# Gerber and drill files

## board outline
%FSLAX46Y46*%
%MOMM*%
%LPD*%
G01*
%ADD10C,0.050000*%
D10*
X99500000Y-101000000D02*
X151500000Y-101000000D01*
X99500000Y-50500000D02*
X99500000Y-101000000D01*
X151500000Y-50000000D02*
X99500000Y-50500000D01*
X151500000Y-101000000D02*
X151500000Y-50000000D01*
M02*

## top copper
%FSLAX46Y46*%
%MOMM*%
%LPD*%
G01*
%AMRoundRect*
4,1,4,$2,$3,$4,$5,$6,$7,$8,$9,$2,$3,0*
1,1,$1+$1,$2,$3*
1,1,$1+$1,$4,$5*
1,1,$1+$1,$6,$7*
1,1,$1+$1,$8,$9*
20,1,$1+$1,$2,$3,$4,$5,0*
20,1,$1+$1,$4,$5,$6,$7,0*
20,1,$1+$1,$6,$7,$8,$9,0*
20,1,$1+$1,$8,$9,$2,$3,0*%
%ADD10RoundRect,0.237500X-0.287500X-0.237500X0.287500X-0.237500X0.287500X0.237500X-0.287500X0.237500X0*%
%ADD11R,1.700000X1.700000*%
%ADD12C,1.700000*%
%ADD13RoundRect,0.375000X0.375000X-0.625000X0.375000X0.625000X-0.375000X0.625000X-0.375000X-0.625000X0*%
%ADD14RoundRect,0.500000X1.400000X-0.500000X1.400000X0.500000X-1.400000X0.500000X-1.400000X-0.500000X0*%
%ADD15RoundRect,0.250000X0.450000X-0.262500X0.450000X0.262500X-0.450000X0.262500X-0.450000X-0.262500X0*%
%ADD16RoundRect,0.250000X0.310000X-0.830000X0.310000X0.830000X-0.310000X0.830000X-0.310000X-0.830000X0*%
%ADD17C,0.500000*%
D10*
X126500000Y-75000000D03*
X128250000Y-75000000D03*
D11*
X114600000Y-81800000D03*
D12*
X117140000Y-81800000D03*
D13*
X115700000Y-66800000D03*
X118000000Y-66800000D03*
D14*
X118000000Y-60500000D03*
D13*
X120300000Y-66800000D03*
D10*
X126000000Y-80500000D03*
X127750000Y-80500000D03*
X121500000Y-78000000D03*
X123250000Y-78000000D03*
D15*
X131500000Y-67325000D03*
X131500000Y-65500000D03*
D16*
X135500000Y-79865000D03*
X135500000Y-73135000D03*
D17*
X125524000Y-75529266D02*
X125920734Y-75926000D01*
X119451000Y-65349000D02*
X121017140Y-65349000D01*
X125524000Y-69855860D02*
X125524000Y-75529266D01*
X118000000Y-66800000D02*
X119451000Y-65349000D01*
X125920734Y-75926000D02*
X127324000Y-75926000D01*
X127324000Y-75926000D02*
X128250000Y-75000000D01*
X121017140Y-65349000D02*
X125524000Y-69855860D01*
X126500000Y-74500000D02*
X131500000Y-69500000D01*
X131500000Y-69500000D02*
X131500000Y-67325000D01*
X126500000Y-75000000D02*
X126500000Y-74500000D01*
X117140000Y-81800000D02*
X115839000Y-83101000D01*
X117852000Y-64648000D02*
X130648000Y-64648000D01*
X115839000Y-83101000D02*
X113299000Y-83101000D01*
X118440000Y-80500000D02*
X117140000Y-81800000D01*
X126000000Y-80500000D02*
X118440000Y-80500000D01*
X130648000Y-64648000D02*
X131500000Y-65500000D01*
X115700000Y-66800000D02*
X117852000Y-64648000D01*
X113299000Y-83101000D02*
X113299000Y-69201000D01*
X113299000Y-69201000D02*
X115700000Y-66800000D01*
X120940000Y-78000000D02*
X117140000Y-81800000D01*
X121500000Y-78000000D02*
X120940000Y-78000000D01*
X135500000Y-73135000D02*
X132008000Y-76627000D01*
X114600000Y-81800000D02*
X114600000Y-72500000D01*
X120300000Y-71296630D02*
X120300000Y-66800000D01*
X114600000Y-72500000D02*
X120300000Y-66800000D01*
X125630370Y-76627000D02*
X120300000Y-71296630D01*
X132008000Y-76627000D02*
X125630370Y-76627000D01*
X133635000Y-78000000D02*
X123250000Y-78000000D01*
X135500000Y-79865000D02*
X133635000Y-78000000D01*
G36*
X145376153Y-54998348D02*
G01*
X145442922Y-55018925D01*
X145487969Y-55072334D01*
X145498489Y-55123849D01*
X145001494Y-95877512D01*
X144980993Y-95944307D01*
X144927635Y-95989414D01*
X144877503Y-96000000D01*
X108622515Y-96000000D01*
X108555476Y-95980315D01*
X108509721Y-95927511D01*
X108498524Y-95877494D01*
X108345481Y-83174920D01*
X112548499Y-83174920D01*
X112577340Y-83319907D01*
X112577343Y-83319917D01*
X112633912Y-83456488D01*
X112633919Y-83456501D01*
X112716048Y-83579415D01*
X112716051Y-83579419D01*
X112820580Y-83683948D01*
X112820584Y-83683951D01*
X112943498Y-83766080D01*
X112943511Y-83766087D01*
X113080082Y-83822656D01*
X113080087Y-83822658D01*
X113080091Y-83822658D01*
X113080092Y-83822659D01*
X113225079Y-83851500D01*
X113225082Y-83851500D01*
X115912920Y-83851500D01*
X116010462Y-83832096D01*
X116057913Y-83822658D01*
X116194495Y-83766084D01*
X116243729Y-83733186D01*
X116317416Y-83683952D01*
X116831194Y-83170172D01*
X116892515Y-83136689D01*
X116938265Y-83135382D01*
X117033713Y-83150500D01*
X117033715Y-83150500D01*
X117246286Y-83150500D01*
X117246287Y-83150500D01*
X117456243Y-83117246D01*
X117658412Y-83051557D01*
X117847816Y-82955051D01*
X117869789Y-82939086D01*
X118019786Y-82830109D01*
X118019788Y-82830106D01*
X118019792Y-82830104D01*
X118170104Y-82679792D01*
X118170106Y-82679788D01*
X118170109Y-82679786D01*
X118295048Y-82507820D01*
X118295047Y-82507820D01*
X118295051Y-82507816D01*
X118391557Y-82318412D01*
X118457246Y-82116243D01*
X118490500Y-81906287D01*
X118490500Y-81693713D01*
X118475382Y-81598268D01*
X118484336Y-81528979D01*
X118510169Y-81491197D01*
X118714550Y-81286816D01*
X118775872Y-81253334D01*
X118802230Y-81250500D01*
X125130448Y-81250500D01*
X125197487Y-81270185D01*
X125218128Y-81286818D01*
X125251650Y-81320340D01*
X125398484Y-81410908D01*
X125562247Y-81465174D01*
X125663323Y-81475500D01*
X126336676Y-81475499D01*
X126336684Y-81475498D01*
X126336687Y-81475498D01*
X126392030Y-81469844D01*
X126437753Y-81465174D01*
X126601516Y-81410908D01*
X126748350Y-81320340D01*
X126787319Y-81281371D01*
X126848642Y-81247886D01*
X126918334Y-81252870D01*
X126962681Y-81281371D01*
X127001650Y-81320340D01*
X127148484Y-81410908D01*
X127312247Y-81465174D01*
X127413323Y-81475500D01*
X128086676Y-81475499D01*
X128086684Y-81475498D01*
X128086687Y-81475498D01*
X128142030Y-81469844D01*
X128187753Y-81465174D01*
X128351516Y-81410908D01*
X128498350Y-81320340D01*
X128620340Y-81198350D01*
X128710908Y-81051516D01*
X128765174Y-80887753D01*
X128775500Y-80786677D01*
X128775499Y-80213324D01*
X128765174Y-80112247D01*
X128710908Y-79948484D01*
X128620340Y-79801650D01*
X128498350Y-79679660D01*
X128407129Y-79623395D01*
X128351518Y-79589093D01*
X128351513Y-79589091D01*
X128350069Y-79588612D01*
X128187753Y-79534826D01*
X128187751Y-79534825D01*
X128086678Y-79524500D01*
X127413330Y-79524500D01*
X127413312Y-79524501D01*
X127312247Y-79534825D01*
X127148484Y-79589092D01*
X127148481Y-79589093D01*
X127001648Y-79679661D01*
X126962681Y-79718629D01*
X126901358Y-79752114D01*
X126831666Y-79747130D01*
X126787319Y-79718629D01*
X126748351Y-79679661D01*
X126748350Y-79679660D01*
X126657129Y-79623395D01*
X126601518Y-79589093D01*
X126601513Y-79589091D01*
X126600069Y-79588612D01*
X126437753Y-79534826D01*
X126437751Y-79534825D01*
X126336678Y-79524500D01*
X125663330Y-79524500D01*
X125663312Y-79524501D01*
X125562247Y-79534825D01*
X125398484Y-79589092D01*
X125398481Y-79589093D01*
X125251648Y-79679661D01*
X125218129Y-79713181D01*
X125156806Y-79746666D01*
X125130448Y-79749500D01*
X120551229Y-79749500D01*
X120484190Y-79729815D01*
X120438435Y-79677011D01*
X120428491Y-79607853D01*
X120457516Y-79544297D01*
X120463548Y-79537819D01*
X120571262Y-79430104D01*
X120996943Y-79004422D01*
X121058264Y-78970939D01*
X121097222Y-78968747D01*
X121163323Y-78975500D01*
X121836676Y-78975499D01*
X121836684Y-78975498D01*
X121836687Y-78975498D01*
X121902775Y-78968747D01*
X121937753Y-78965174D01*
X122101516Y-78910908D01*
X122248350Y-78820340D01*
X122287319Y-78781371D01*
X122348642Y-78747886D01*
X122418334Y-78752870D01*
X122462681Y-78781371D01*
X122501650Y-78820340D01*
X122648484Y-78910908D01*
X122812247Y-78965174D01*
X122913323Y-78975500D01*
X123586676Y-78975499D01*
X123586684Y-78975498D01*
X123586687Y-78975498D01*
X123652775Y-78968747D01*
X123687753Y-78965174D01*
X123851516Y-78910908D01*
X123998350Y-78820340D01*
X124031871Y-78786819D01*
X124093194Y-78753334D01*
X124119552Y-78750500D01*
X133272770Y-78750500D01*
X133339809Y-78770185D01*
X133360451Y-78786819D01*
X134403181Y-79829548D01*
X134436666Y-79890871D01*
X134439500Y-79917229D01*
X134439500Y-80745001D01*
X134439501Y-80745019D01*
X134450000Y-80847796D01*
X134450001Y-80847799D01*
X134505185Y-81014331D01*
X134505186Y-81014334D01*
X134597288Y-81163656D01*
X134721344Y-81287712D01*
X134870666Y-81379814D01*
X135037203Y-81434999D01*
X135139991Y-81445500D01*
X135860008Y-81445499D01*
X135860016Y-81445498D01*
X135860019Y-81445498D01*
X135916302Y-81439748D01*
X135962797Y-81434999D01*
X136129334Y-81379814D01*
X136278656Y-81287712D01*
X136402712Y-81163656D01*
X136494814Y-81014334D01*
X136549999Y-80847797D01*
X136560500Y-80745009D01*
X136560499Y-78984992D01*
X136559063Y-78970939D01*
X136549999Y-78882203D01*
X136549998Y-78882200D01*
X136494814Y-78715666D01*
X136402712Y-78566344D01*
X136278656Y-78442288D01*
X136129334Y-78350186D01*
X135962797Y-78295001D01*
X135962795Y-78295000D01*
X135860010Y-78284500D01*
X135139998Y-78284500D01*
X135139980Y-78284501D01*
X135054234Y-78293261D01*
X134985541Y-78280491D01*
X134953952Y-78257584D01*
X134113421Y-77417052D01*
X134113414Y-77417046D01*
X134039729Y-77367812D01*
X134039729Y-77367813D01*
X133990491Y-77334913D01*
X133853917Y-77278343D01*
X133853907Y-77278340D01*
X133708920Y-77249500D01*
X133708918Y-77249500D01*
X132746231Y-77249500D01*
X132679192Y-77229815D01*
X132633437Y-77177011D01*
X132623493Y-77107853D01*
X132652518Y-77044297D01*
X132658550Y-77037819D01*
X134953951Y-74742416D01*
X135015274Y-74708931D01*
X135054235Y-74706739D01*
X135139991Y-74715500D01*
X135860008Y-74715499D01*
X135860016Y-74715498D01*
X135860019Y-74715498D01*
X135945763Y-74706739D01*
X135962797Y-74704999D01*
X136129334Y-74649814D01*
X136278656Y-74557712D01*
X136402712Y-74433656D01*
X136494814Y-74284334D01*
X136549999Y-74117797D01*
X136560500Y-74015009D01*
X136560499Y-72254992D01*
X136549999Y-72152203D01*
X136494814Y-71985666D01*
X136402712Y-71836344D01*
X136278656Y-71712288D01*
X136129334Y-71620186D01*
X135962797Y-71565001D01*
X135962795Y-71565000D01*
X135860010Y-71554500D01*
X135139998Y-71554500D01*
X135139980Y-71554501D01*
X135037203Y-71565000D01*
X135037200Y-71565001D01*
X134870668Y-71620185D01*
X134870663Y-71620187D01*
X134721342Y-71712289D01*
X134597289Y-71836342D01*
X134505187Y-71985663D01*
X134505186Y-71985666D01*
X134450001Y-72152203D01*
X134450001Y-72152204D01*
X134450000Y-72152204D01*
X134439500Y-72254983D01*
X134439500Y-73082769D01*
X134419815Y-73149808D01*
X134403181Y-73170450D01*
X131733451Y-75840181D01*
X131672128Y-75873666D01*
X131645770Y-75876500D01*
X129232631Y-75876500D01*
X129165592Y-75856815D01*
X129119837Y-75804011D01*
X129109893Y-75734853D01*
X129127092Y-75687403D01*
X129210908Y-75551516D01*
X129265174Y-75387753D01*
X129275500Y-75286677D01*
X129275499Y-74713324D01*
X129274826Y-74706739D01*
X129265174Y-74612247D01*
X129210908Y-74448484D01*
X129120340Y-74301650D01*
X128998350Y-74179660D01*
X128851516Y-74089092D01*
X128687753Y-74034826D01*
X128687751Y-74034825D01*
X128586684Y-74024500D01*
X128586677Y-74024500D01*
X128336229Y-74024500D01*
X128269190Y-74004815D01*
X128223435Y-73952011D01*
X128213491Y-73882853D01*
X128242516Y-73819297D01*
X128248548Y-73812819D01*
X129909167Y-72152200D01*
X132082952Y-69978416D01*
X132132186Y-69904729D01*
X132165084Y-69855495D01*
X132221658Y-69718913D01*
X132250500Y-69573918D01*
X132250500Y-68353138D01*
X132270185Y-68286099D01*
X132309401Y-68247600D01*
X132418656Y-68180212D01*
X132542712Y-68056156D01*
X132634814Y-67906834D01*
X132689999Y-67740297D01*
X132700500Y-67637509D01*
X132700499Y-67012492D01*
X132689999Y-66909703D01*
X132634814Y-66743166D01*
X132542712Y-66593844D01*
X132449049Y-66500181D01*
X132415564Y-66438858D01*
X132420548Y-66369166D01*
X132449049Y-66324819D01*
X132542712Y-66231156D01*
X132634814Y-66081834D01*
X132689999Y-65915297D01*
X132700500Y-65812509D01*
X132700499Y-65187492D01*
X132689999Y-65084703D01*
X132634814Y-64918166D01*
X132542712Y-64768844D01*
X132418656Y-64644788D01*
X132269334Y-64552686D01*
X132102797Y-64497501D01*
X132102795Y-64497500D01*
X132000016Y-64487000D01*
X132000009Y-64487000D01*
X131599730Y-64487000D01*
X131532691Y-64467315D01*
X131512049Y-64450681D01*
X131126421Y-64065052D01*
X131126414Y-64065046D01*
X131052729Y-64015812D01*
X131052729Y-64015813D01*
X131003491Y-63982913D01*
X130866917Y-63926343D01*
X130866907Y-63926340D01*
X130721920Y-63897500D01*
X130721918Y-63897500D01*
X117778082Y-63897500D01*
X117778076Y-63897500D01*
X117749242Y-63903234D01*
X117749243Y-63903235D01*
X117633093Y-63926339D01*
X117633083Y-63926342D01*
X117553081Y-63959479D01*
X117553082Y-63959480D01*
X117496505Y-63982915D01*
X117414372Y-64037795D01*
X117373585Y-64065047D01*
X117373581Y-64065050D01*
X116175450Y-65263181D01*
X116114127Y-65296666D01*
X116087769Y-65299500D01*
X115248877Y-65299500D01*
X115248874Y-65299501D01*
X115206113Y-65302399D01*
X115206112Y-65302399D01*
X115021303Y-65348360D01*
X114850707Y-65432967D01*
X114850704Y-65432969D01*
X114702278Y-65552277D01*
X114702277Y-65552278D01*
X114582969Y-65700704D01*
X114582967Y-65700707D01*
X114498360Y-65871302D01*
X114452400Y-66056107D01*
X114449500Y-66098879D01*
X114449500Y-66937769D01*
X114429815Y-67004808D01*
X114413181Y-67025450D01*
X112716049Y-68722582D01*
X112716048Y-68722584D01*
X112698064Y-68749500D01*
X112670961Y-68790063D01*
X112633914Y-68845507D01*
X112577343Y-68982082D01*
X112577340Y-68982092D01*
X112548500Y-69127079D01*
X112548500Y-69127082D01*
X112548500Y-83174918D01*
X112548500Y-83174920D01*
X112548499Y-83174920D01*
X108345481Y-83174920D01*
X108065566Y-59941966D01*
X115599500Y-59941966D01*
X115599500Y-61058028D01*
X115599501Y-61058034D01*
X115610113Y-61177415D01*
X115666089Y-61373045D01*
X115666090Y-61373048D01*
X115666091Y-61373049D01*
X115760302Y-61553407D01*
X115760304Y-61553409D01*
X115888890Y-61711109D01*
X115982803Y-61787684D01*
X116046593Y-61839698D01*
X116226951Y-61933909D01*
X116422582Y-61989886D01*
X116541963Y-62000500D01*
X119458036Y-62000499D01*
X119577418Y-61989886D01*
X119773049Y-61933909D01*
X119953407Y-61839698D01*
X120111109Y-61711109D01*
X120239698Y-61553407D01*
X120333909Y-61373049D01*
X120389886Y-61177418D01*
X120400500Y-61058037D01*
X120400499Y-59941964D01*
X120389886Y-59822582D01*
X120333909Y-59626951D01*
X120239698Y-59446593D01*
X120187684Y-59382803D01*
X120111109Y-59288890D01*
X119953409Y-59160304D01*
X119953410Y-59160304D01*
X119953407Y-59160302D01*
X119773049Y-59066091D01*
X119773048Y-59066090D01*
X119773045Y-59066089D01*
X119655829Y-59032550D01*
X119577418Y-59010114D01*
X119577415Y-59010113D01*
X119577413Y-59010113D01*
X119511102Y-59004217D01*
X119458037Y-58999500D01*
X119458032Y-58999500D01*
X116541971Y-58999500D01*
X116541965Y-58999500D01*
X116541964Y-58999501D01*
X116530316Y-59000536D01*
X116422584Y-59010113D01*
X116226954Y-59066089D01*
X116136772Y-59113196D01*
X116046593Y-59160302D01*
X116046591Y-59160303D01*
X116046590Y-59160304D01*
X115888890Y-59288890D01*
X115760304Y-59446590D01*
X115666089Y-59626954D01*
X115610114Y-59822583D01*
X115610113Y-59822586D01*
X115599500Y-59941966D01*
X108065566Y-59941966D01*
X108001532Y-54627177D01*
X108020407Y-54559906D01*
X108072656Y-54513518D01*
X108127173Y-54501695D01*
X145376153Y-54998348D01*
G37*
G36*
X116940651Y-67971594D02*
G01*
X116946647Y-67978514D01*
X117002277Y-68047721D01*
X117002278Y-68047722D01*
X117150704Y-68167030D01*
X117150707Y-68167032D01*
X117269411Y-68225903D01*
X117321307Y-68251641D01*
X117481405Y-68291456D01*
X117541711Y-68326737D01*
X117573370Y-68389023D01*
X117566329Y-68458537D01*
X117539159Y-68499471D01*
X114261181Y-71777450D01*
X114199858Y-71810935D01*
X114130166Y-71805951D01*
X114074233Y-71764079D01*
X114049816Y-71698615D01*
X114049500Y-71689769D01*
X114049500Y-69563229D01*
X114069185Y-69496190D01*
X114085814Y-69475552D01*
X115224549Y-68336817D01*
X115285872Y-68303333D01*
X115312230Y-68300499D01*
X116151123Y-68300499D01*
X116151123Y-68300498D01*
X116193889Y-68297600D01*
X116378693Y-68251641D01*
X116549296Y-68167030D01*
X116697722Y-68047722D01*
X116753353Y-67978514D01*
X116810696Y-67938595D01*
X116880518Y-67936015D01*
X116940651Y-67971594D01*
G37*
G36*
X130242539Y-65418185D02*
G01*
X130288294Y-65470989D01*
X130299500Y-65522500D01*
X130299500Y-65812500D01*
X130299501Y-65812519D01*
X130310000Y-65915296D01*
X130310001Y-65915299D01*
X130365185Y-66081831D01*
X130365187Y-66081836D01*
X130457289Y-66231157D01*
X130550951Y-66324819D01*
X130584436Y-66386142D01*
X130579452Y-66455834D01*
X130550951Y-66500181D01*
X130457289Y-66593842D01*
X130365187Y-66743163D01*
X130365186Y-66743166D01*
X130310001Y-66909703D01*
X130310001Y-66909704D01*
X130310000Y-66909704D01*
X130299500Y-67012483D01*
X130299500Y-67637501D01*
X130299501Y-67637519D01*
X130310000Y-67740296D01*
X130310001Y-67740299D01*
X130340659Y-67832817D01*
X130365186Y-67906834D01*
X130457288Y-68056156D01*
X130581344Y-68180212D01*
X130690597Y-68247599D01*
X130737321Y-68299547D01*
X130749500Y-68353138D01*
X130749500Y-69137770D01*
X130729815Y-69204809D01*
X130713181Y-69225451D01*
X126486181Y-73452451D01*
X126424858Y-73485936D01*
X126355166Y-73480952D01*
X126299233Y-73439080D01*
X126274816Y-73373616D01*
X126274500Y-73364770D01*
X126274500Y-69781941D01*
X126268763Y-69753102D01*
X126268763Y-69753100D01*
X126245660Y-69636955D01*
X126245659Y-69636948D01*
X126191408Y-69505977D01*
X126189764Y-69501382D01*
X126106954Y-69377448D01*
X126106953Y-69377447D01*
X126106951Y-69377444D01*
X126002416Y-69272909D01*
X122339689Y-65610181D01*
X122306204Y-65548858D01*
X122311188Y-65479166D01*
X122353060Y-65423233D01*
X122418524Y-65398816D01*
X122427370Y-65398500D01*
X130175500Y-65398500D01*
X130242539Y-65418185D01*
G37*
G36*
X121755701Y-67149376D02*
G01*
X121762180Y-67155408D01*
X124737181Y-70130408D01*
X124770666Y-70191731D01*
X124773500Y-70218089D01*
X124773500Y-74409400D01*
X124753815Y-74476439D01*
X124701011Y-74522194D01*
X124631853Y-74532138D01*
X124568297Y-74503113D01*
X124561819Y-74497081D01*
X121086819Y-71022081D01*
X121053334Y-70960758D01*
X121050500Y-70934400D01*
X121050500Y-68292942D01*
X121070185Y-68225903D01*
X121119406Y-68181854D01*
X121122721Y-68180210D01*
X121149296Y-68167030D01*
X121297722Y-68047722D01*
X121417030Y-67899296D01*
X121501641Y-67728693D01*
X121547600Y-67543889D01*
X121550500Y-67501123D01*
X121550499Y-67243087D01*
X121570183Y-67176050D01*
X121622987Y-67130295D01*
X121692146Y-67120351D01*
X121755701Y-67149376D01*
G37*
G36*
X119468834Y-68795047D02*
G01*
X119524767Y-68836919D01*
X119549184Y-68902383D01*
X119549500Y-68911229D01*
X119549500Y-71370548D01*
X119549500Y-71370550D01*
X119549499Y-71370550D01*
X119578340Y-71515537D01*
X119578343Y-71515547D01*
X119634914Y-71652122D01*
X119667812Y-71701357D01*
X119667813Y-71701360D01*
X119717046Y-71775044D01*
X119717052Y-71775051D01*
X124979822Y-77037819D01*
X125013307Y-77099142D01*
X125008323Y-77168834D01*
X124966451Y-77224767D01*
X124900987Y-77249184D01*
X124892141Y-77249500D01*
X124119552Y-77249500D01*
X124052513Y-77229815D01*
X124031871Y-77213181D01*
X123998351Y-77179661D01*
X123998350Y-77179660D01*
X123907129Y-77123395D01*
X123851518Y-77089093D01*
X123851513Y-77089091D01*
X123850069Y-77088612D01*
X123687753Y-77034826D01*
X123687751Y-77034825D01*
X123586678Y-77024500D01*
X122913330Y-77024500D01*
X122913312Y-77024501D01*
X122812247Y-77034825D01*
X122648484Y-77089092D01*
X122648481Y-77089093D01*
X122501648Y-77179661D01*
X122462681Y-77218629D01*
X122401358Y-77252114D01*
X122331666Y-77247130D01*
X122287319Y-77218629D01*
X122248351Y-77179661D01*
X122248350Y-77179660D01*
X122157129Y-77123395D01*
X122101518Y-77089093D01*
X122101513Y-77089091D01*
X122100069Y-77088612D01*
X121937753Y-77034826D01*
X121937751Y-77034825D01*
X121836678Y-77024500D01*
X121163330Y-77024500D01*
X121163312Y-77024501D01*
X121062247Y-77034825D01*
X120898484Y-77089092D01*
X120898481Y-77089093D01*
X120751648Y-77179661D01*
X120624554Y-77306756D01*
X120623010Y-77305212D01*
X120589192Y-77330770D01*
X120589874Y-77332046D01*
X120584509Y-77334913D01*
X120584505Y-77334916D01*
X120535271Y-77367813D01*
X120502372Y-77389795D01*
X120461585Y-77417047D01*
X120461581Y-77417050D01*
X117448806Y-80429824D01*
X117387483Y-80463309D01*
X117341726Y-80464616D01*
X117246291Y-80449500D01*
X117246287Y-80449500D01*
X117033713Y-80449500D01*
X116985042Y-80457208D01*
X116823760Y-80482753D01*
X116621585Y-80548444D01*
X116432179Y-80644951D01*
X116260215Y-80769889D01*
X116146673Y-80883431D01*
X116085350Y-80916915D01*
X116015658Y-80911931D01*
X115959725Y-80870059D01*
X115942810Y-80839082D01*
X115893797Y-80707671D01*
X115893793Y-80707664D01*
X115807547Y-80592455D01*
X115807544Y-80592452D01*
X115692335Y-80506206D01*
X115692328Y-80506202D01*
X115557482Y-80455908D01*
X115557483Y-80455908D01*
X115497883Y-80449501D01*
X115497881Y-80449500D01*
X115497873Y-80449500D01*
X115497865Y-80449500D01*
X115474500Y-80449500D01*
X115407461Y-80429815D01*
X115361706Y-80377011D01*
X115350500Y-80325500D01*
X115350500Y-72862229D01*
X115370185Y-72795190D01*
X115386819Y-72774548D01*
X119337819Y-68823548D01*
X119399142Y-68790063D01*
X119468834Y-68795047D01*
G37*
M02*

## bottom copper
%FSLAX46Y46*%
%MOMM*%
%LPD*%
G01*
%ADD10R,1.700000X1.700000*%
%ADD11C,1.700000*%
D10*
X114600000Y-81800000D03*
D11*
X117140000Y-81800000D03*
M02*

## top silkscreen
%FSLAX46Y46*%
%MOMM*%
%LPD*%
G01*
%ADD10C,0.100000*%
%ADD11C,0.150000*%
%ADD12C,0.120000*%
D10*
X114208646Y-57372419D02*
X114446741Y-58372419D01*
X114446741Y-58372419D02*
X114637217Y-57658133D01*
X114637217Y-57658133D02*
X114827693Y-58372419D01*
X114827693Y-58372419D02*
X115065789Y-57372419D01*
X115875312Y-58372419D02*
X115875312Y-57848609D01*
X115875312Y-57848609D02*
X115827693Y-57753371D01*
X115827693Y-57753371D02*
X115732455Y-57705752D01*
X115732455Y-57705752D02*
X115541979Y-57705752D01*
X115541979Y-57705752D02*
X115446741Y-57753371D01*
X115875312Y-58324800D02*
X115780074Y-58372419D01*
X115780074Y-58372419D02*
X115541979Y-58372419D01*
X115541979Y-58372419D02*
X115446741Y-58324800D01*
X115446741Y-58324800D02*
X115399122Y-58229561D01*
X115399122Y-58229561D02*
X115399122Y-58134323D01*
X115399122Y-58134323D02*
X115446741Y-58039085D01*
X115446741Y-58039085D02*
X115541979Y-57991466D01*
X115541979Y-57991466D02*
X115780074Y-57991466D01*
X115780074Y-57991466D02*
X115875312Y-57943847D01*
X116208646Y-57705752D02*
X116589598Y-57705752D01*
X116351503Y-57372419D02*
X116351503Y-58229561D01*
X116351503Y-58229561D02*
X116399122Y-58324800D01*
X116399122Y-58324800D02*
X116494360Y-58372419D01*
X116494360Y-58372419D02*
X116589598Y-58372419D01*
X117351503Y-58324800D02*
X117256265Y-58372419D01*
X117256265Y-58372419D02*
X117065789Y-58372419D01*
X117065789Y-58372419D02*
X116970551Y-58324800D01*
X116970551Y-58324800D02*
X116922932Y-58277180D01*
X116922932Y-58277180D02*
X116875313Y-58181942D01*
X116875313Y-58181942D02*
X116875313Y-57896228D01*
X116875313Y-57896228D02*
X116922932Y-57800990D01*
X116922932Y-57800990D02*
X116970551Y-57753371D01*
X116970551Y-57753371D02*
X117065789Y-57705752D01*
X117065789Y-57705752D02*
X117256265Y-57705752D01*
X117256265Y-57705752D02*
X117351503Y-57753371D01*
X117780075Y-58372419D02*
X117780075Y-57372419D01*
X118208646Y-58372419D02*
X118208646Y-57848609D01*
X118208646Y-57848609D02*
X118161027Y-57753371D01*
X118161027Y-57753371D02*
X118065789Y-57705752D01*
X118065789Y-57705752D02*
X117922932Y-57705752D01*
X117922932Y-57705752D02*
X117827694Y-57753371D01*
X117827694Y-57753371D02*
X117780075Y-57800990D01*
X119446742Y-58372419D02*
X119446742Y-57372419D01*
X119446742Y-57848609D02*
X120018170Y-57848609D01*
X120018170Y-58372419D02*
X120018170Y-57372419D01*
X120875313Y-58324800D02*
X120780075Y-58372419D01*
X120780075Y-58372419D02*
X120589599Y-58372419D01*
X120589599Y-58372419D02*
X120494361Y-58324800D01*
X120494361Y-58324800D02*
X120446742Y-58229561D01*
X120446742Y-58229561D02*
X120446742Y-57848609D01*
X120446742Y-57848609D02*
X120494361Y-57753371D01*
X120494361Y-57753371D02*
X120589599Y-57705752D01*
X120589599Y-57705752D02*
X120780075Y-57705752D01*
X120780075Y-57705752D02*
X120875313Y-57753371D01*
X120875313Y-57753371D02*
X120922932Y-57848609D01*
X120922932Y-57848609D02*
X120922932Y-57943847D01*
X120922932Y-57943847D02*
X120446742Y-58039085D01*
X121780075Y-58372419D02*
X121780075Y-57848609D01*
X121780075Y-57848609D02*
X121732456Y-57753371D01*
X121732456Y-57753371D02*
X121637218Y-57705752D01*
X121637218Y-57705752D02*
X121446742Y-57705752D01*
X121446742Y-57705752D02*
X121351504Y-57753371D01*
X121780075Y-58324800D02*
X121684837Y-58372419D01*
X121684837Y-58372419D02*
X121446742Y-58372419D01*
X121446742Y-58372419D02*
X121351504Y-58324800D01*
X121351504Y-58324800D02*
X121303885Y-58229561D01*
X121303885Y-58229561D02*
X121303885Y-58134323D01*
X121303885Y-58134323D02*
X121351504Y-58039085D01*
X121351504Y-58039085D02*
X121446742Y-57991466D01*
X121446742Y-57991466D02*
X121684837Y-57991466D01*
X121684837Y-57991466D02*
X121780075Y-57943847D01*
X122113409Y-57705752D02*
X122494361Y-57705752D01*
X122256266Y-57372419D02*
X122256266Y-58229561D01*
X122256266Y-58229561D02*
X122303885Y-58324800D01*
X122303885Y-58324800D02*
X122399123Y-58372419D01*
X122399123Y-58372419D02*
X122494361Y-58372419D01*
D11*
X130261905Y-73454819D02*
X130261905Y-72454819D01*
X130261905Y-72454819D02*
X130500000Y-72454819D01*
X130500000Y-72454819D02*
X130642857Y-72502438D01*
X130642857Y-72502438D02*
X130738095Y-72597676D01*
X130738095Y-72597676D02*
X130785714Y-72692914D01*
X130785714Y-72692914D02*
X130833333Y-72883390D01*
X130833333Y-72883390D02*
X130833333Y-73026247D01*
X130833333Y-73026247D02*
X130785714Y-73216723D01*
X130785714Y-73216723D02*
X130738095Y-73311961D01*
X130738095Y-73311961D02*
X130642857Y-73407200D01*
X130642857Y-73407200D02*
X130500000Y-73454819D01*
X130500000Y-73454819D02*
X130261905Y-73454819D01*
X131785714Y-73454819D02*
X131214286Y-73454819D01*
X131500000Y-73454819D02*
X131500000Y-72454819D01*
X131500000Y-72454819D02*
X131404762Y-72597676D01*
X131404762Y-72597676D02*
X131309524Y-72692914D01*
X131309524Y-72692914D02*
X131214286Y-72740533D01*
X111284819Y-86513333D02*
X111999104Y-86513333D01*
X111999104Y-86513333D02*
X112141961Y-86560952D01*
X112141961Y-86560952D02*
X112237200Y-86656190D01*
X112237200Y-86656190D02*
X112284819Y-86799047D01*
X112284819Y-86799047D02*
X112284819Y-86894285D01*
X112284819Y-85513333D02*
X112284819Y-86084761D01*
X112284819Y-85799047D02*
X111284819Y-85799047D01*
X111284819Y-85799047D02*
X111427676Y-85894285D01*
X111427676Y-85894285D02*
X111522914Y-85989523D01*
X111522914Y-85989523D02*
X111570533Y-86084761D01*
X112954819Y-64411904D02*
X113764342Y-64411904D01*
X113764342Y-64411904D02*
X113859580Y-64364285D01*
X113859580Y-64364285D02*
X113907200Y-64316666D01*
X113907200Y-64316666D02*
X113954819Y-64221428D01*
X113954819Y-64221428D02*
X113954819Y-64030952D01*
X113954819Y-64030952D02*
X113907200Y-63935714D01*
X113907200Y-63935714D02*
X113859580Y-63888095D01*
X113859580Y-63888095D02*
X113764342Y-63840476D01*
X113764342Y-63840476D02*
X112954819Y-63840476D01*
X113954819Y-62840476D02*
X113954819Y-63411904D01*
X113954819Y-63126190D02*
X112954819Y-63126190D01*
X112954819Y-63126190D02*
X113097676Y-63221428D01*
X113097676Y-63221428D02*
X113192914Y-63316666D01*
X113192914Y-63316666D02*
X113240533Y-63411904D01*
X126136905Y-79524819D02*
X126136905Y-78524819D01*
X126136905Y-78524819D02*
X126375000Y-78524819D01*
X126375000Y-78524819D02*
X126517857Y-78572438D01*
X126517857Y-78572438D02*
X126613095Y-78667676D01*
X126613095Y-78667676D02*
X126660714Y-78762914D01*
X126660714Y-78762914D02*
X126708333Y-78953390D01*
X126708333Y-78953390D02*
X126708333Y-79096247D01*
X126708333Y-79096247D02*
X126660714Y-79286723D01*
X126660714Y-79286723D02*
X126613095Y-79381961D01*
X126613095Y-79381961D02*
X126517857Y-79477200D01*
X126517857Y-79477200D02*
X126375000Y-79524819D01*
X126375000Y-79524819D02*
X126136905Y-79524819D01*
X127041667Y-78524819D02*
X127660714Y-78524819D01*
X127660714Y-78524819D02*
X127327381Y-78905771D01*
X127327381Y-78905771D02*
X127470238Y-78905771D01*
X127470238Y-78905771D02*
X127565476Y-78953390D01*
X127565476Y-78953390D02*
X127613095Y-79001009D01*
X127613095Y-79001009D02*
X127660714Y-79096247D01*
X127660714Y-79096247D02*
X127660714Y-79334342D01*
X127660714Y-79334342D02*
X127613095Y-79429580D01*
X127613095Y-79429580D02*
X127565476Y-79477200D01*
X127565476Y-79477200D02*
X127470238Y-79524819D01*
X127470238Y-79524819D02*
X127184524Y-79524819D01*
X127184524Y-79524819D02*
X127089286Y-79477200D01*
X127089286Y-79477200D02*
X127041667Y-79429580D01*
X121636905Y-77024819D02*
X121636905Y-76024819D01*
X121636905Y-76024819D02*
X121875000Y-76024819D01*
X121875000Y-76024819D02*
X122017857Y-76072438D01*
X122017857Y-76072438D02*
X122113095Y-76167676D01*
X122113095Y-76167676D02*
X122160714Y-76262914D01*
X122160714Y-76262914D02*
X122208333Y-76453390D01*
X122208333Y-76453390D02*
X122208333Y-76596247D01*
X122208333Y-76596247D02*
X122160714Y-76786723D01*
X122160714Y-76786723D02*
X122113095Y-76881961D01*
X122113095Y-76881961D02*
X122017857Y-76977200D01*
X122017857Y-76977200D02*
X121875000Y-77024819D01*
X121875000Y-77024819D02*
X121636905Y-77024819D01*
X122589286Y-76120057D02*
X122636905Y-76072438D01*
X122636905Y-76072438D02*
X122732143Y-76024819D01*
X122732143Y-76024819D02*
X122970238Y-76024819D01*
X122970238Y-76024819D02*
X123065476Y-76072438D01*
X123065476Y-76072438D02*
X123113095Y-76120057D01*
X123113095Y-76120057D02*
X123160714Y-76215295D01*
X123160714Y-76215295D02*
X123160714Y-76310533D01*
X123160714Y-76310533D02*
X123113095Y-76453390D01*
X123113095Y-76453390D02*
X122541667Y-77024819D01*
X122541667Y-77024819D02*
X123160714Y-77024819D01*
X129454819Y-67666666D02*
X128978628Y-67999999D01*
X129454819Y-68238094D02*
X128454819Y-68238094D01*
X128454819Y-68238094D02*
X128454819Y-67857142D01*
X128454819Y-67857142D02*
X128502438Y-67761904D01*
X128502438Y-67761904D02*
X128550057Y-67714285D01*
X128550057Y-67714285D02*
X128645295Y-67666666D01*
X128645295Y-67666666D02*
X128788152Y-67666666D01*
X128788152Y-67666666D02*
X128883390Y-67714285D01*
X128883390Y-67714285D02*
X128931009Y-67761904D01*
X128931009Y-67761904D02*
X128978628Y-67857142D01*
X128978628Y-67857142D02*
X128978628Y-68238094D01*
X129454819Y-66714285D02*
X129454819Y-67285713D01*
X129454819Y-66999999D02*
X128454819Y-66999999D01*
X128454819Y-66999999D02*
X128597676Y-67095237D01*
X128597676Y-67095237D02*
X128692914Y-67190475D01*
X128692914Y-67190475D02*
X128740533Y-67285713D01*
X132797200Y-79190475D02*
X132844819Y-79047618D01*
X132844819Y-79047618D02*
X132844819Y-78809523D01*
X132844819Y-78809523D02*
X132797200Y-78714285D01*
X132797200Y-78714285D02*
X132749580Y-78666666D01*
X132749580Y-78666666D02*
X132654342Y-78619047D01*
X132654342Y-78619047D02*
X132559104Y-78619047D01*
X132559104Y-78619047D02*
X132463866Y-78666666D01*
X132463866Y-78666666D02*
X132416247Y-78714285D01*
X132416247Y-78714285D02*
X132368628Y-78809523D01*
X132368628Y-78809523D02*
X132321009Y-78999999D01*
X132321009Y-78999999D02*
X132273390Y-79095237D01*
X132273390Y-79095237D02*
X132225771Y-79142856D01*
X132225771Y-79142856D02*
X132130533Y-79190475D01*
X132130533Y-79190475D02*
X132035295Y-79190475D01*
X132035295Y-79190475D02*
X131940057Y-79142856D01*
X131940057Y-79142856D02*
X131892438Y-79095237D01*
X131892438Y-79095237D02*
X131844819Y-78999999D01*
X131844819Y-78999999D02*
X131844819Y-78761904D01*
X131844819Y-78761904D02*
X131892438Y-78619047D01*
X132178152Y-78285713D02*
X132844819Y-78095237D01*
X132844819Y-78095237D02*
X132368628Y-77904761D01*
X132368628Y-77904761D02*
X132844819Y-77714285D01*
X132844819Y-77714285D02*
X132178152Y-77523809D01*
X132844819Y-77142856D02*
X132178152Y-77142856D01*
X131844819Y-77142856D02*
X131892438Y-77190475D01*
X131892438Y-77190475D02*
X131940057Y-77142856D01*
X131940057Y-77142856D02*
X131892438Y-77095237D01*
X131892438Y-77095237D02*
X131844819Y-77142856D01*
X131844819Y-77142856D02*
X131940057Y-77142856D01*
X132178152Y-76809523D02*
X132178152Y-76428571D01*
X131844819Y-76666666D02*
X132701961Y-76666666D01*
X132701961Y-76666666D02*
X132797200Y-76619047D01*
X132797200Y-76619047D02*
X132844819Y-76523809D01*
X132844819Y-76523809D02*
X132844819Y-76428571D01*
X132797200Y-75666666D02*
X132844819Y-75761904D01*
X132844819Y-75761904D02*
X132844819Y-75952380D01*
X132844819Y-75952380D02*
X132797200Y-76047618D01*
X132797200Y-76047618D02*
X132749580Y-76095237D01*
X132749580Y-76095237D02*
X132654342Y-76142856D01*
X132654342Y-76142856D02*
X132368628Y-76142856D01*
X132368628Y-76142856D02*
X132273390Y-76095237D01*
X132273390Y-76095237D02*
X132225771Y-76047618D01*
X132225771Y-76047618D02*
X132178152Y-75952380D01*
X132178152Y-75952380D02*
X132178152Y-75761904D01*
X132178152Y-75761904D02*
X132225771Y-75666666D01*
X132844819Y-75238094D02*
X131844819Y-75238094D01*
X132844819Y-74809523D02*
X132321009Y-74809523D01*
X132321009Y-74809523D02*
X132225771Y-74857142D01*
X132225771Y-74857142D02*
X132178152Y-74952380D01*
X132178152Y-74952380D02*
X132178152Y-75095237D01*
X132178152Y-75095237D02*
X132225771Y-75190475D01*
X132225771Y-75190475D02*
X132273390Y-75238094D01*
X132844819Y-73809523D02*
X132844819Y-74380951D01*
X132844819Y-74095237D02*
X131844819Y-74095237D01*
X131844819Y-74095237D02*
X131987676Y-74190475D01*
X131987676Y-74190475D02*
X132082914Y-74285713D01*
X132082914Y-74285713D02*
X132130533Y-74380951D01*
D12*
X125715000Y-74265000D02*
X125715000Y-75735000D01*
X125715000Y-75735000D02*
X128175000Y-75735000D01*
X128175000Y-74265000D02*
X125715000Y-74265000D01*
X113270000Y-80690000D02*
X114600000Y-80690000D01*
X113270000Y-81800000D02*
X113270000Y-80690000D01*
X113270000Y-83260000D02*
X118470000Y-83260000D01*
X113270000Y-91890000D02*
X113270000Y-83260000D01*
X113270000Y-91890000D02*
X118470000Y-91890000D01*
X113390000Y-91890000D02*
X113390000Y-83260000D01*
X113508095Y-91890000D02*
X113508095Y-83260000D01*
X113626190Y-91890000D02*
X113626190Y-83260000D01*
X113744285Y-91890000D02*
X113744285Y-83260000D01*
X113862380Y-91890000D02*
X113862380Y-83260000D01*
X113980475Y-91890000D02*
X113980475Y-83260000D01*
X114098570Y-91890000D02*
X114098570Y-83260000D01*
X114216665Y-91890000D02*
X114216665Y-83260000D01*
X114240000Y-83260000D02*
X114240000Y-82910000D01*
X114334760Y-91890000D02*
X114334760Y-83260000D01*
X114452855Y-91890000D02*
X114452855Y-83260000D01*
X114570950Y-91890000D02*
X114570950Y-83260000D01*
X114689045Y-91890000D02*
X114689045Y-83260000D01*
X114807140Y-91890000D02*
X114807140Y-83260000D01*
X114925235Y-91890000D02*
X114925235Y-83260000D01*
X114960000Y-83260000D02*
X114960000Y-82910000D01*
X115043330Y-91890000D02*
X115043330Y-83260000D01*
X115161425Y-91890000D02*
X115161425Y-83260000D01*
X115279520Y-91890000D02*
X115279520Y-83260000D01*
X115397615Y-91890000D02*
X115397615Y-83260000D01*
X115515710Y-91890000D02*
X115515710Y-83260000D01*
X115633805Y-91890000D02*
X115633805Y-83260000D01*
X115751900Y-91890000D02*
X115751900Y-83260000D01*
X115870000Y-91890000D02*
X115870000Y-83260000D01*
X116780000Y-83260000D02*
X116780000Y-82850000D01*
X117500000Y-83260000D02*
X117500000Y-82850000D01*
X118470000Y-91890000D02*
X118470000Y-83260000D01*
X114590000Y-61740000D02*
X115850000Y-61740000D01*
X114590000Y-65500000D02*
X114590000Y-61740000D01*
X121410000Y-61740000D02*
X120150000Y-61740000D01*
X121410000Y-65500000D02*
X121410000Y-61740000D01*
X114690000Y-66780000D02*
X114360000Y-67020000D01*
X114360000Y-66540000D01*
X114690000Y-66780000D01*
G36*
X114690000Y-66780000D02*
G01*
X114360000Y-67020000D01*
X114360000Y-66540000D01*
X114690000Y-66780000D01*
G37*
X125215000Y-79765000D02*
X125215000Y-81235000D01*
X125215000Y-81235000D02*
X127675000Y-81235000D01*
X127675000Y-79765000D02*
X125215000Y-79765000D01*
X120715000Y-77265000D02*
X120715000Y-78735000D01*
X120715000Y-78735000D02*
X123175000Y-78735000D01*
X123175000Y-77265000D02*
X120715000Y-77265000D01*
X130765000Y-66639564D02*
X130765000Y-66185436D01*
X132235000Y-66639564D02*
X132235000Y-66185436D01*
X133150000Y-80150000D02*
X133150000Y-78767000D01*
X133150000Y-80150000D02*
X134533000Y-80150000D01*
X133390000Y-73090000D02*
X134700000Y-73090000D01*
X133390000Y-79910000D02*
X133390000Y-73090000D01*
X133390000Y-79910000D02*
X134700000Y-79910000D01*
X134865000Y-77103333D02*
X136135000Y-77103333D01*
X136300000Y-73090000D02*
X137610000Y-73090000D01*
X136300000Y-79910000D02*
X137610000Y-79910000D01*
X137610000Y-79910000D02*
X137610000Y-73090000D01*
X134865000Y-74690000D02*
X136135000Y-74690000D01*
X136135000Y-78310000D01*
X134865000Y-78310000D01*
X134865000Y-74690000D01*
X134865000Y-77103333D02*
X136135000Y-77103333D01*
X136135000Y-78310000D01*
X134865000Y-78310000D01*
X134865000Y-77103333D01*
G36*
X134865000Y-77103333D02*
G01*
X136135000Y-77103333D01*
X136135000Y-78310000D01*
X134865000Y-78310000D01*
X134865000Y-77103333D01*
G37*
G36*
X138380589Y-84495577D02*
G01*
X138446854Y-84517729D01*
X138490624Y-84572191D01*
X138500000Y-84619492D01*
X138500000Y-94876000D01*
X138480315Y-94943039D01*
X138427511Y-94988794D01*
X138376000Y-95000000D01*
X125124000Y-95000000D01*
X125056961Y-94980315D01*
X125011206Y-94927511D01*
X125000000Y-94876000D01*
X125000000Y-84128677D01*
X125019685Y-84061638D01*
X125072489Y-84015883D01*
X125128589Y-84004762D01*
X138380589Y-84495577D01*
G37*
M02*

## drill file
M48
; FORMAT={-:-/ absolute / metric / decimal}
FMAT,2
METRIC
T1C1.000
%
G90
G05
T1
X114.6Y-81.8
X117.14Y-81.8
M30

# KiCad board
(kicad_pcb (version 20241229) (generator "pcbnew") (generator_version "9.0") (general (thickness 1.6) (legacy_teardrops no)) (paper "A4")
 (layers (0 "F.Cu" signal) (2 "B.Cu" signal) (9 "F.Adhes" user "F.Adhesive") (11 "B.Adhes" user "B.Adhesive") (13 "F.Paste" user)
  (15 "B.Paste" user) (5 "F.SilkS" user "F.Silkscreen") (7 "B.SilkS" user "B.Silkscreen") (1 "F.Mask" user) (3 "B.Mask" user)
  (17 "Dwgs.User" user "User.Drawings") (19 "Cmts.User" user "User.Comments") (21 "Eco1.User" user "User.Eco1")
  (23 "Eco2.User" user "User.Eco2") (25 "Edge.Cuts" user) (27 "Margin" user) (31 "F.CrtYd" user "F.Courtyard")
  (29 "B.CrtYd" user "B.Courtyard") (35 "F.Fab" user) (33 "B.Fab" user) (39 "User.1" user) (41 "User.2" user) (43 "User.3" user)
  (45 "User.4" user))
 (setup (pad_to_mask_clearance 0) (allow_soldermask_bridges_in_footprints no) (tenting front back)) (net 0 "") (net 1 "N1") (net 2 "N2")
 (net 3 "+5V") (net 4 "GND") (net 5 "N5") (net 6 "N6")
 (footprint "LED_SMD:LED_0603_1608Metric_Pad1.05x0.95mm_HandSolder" (layer "F.Cu") (at 127.375 75)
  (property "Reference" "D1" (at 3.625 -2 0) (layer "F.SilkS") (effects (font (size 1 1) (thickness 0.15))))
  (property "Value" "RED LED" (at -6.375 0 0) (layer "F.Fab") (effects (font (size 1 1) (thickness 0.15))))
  (fp_line (start -1.66 -0.735) (end -1.66 0.735) (stroke (width 0.12) (type solid)) (layer "F.SilkS"))
  (fp_line (start -1.66 0.735) (end 0.8 0.735) (stroke (width 0.12) (type solid)) (layer "F.SilkS"))
  (fp_line (start 0.8 -0.735) (end -1.66 -0.735) (stroke (width 0.12) (type solid)) (layer "F.SilkS"))
  (pad "1" smd roundrect (at -0.875 0) (size 1.05 0.95) (layers "F.Cu" "F.Mask" "F.Paste") (roundrect_rratio 0.25) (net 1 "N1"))
  (pad "2" smd roundrect (at 0.875 0) (size 1.05 0.95) (layers "F.Cu" "F.Mask" "F.Paste") (roundrect_rratio 0.25) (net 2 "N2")))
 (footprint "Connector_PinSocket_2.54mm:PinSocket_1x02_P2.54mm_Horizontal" (layer "F.Cu") (at 114.6 81.8 90)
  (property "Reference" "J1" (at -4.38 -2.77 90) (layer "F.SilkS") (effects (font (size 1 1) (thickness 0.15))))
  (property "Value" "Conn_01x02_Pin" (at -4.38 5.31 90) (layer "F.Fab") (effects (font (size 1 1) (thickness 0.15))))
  (fp_line (start 1.11 -1.33) (end 1.11 0) (stroke (width 0.12) (type solid)) (layer "F.SilkS"))
  (fp_line (start 0 -1.33) (end 1.11 -1.33) (stroke (width 0.12) (type solid)) (layer "F.SilkS"))
  (fp_line (start -1.46 -1.33) (end -1.46 3.87) (stroke (width 0.12) (type solid)) (layer "F.SilkS"))
  (fp_line (start -10.09 -1.33) (end -1.46 -1.33) (stroke (width 0.12) (type solid)) (layer "F.SilkS"))
  (fp_line (start -10.09 -1.33) (end -10.09 3.87) (stroke (width 0.12) (type solid)) (layer "F.SilkS"))
  (fp_line (start -10.09 -1.21) (end -1.46 -1.21) (stroke (width 0.12) (type solid)) (layer "F.SilkS"))
  (fp_line (start -10.09 -1.091905) (end -1.46 -1.091905) (stroke (width 0.12) (type solid)) (layer "F.SilkS"))
  (fp_line (start -10.09 -0.97381) (end -1.46 -0.97381) (stroke (width 0.12) (type solid)) (layer "F.SilkS"))
  (fp_line (start -10.09 -0.855715) (end -1.46 -0.855715) (stroke (width 0.12) (type solid)) (layer "F.SilkS"))
  (fp_line (start -10.09 -0.73762) (end -1.46 -0.73762) (stroke (width 0.12) (type solid)) (layer "F.SilkS"))
  (fp_line (start -10.09 -0.619525) (end -1.46 -0.619525) (stroke (width 0.12) (type solid)) (layer "F.SilkS"))
  (fp_line (start -10.09 -0.50143) (end -1.46 -0.50143) (stroke (width 0.12) (type solid)) (layer "F.SilkS"))
  (fp_line (start -10.09 -0.383335) (end -1.46 -0.383335) (stroke (width 0.12) (type solid)) (layer "F.SilkS"))
  (fp_line (start -1.46 -0.36) (end -1.11 -0.36) (stroke (width 0.12) (type solid)) (layer "F.SilkS"))
  (fp_line (start -10.09 -0.26524) (end -1.46 -0.26524) (stroke (width 0.12) (type solid)) (layer "F.SilkS"))
  (fp_line (start -10.09 -0.147145) (end -1.46 -0.147145) (stroke (width 0.12) (type solid)) (layer "F.SilkS"))
  (fp_line (start -10.09 -0.02905) (end -1.46 -0.02905) (stroke (width 0.12) (type solid)) (layer "F.SilkS"))
  (fp_line (start -10.09 0.089045) (end -1.46 0.089045) (stroke (width 0.12) (type solid)) (layer "F.SilkS"))
  (fp_line (start -10.09 0.20714) (end -1.46 0.20714) (stroke (width 0.12) (type solid)) (layer "F.SilkS"))
  (fp_line (start -10.09 0.325235) (end -1.46 0.325235) (stroke (width 0.12) (type solid)) (layer "F.SilkS"))
  (fp_line (start -1.46 0.36) (end -1.11 0.36) (stroke (width 0.12) (type solid)) (layer "F.SilkS"))
  (fp_line (start -10.09 0.44333) (end -1.46 0.44333) (stroke (width 0.12) (type solid)) (layer "F.SilkS"))
  (fp_line (start -10.09 0.561425) (end -1.46 0.561425) (stroke (width 0.12) (type solid)) (layer "F.SilkS"))
  (fp_line (start -10.09 0.67952) (end -1.46 0.67952) (stroke (width 0.12) (type solid)) (layer "F.SilkS"))
  (fp_line (start -10.09 0.797615) (end -1.46 0.797615) (stroke (width 0.12) (type solid)) (layer "F.SilkS"))
  (fp_line (start -10.09 0.91571) (end -1.46 0.91571) (stroke (width 0.12) (type solid)) (layer "F.SilkS"))
  (fp_line (start -10.09 1.033805) (end -1.46 1.033805) (stroke (width 0.12) (type solid)) (layer "F.SilkS"))
  (fp_line (start -10.09 1.1519) (end -1.46 1.1519) (stroke (width 0.12) (type solid)) (layer "F.SilkS"))
  (fp_line (start -10.09 1.27) (end -1.46 1.27) (stroke (width 0.12) (type solid)) (layer "F.SilkS"))
  (fp_line (start -1.46 2.18) (end -1.05 2.18) (stroke (width 0.12) (type solid)) (layer "F.SilkS"))
  (fp_line (start -1.46 2.9) (end -1.05 2.9) (stroke (width 0.12) (type solid)) (layer "F.SilkS"))
  (fp_line (start -10.09 3.87) (end -1.46 3.87) (stroke (width 0.12) (type solid)) (layer "F.SilkS"))
  (pad "1" thru_hole rect (at 0 0 90) (size 1.7 1.7) (drill 1) (layers "*.Cu" "*.Mask") (remove_unused_layers no) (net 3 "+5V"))
  (pad "2" thru_hole circle (at 0 2.54 90) (size 1.7 1.7) (drill 1) (layers "*.Cu" "*.Mask") (remove_unused_layers no) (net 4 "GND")))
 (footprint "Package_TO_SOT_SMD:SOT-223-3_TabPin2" (layer "F.Cu") (at 118 63.65 90)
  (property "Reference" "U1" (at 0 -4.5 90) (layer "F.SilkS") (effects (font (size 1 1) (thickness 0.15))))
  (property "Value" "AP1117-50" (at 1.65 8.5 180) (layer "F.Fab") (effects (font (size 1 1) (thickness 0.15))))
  (fp_line (start 1.91 -3.41) (end 1.91 -2.15) (stroke (width 0.12) (type solid)) (layer "F.SilkS"))
  (fp_line (start -1.85 -3.41) (end 1.91 -3.41) (stroke (width 0.12) (type solid)) (layer "F.SilkS"))
  (fp_line (start 1.91 3.41) (end 1.91 2.15) (stroke (width 0.12) (type solid)) (layer "F.SilkS"))
  (fp_line (start -1.85 3.41) (end 1.91 3.41) (stroke (width 0.12) (type solid)) (layer "F.SilkS"))
  (fp_poly
   (pts (xy -3.13 -3.31) (xy -3.37 -3.64) (xy -2.89 -3.64) (xy -3.13 -3.31)) (stroke (width 0.12) (type solid)) (fill yes) (layer "F.SilkS"))
  (pad "1" smd roundrect (at -3.15 -2.3 90) (size 2 1.5) (layers "F.Cu" "F.Mask" "F.Paste") (roundrect_rratio 0.25) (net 4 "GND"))
  (pad "2" smd roundrect (at -3.15 0 90) (size 2 1.5) (layers "F.Cu" "F.Mask" "F.Paste") (roundrect_rratio 0.25) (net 2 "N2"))
  (pad "2" smd roundrect (at 3.15 0 90) (size 2 3.8) (layers "F.Cu" "F.Mask" "F.Paste") (roundrect_rratio 0.25) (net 2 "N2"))
  (pad "3" smd roundrect (at -3.15 2.3 90) (size 2 1.5) (layers "F.Cu" "F.Mask" "F.Paste") (roundrect_rratio 0.25) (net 3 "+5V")))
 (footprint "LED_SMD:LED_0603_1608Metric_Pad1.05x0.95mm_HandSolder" (layer "F.Cu") (at 126.875 80.5)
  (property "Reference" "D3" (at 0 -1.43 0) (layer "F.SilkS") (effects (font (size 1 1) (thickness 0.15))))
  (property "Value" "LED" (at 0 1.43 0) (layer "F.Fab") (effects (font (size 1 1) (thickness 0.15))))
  (fp_line (start -1.66 -0.735) (end -1.66 0.735) (stroke (width 0.12) (type solid)) (layer "F.SilkS"))
  (fp_line (start -1.66 0.735) (end 0.8 0.735) (stroke (width 0.12) (type solid)) (layer "F.SilkS"))
  (fp_line (start 0.8 -0.735) (end -1.66 -0.735) (stroke (width 0.12) (type solid)) (layer "F.SilkS"))
  (pad "1" smd roundrect (at -0.875 0) (size 1.05 0.95) (layers "F.Cu" "F.Mask" "F.Paste") (roundrect_rratio 0.25) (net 4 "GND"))
  (pad "2" smd roundrect (at 0.875 0) (size 1.05 0.95) (layers "F.Cu" "F.Mask" "F.Paste") (roundrect_rratio 0.25) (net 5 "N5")))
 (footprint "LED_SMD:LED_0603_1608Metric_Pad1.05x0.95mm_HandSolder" (layer "F.Cu") (at 122.375 78)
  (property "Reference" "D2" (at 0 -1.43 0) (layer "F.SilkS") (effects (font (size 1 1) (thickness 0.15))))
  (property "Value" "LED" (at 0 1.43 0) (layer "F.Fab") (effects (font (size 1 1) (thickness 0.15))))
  (fp_line (start -1.66 -0.735) (end -1.66 0.735) (stroke (width 0.12) (type solid)) (layer "F.SilkS"))
  (fp_line (start -1.66 0.735) (end 0.8 0.735) (stroke (width 0.12) (type solid)) (layer "F.SilkS"))
  (fp_line (start 0.8 -0.735) (end -1.66 -0.735) (stroke (width 0.12) (type solid)) (layer "F.SilkS"))
  (pad "1" smd roundrect (at -0.875 0) (size 1.05 0.95) (layers "F.Cu" "F.Mask" "F.Paste") (roundrect_rratio 0.25) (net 4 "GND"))
  (pad "2" smd roundrect (at 0.875 0) (size 1.05 0.95) (layers "F.Cu" "F.Mask" "F.Paste") (roundrect_rratio 0.25) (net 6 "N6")))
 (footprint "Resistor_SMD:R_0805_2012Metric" (layer "F.Cu") (at 131.5 66.4125 90)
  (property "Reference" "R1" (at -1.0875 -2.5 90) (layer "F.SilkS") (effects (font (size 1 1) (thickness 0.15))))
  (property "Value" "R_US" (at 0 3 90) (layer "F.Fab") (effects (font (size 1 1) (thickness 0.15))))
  (fp_line (start -0.227064 -0.735) (end 0.227064 -0.735) (stroke (width 0.12) (type solid)) (layer "F.SilkS"))
  (fp_line (start -0.227064 0.735) (end 0.227064 0.735) (stroke (width 0.12) (type solid)) (layer "F.SilkS"))
  (pad "1" smd roundrect (at -0.9125 0 90) (size 1.025 1.4) (layers "F.Cu" "F.Mask" "F.Paste") (roundrect_rratio 0.243902) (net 1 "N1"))
  (pad "2" smd roundrect (at 0.9125 0 90) (size 1.025 1.4) (layers "F.Cu" "F.Mask" "F.Paste") (roundrect_rratio 0.243902) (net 4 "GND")))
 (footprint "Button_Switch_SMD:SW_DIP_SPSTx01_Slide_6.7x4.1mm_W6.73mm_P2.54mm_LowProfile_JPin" (layer "F.Cu") (at 135.5 76.5 90)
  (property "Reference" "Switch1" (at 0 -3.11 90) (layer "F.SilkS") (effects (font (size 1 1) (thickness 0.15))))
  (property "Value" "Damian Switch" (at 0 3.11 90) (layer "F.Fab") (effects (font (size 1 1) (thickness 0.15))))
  (fp_line (start -3.65 -2.35) (end -2.267 -2.35) (stroke (width 0.12) (type solid)) (layer "F.SilkS"))
  (fp_line (start -3.65 -2.35) (end -3.65 -0.967) (stroke (width 0.12) (type solid)) (layer "F.SilkS"))
  (fp_line (start 3.41 -2.11) (end 3.41 -0.8) (stroke (width 0.12) (type solid)) (layer "F.SilkS"))
  (fp_line (start -3.41 -2.11) (end 3.41 -2.11) (stroke (width 0.12) (type solid)) (layer "F.SilkS"))
  (fp_line (start -3.41 -2.11) (end -3.41 -0.8) (stroke (width 0.12) (type solid)) (layer "F.SilkS"))
  (fp_line (start -0.603333 -0.635) (end -0.603333 0.635) (stroke (width 0.12) (type solid)) (layer "F.SilkS"))
  (fp_line (start 3.41 0.8) (end 3.41 2.11) (stroke (width 0.12) (type solid)) (layer "F.SilkS"))
  (fp_line (start -3.41 0.8) (end -3.41 2.11) (stroke (width 0.12) (type solid)) (layer "F.SilkS"))
  (fp_line (start -3.41 2.11) (end 3.41 2.11) (stroke (width 0.12) (type solid)) (layer "F.SilkS"))
  (fp_rect (start -1.81 -0.635) (end 1.81 0.635) (stroke (width 0.12) (type solid)) (fill no) (layer "F.SilkS"))
  (fp_rect (start -1.81 -0.635) (end -0.603333 0.635) (stroke (width 0.12) (type solid)) (fill yes) (layer "F.SilkS"))
  (pad "1" smd roundrect (at -3.365 0 90) (size 2.16 1.12) (layers "F.Cu" "F.Mask" "F.Paste") (roundrect_rratio 0.223214) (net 6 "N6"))
  (pad "2" smd roundrect (at 3.365 0 90) (size 2.16 1.12) (layers "F.Cu" "F.Mask" "F.Paste") (roundrect_rratio 0.223214) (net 3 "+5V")))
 (gr_line (start 99.5 101) (end 151.5 101) (stroke (width 0.05) (type default)) (layer "Edge.Cuts"))
 (gr_line (start 99.5 50.5) (end 99.5 101) (stroke (width 0.05) (type default)) (layer "Edge.Cuts"))
 (gr_line (start 151.5 50) (end 99.5 50.5) (stroke (width 0.05) (type default)) (layer "Edge.Cuts"))
 (gr_line (start 151.5 101) (end 151.5 50) (stroke (width 0.05) (type default)) (layer "Edge.Cuts"))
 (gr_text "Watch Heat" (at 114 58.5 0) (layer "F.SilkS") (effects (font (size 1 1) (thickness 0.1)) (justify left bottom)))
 (segment (start 125.524 75.529266) (end 125.920734 75.926) (width 0.5) (layer "F.Cu") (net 2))
 (segment (start 119.451 65.349) (end 121.01714 65.349) (width 0.5) (layer "F.Cu") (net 2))
 (segment (start 125.524 69.85586) (end 125.524 75.529266) (width 0.5) (layer "F.Cu") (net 2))
 (segment (start 118 66.8) (end 119.451 65.349) (width 0.5) (layer "F.Cu") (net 2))
 (segment (start 125.920734 75.926) (end 127.324 75.926) (width 0.5) (layer "F.Cu") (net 2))
 (segment (start 127.324 75.926) (end 128.25 75) (width 0.5) (layer "F.Cu") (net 2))
 (segment (start 121.01714 65.349) (end 125.524 69.85586) (width 0.5) (layer "F.Cu") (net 2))
 (segment (start 126.5 74.5) (end 131.5 69.5) (width 0.5) (layer "F.Cu") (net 1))
 (segment (start 131.5 69.5) (end 131.5 67.325) (width 0.5) (layer "F.Cu") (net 1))
 (segment (start 126.5 75) (end 126.5 74.5) (width 0.5) (layer "F.Cu") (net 1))
 (segment (start 117.14 81.8) (end 115.839 83.101) (width 0.5) (layer "F.Cu") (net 4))
 (segment (start 117.852 64.648) (end 130.648 64.648) (width 0.5) (layer "F.Cu") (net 4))
 (segment (start 115.839 83.101) (end 113.299 83.101) (width 0.5) (layer "F.Cu") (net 4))
 (segment (start 118.44 80.5) (end 117.14 81.8) (width 0.5) (layer "F.Cu") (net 4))
 (segment (start 126 80.5) (end 118.44 80.5) (width 0.5) (layer "F.Cu") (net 4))
 (segment (start 130.648 64.648) (end 131.5 65.5) (width 0.5) (layer "F.Cu") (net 4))
 (segment (start 115.7 66.8) (end 117.852 64.648) (width 0.5) (layer "F.Cu") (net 4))
 (segment (start 113.299 83.101) (end 113.299 69.201) (width 0.5) (layer "F.Cu") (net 4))
 (segment (start 113.299 69.201) (end 115.7 66.8) (width 0.5) (layer "F.Cu") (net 4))
 (segment (start 120.94 78) (end 117.14 81.8) (width 0.5) (layer "F.Cu") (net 4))
 (segment (start 121.5 78) (end 120.94 78) (width 0.5) (layer "F.Cu") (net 4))
 (segment (start 135.5 73.135) (end 132.008 76.627) (width 0.5) (layer "F.Cu") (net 3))
 (segment (start 114.6 81.8) (end 114.6 72.5) (width 0.5) (layer "F.Cu") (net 3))
 (segment (start 120.3 71.29663) (end 120.3 66.8) (width 0.5) (layer "F.Cu") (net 3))
 (segment (start 114.6 72.5) (end 120.3 66.8) (width 0.5) (layer "F.Cu") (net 3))
 (segment (start 125.63037 76.627) (end 120.3 71.29663) (width 0.5) (layer "F.Cu") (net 3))
 (segment (start 132.008 76.627) (end 125.63037 76.627) (width 0.5) (layer "F.Cu") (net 3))
 (segment (start 133.635 78) (end 123.25 78) (width 0.5) (layer "F.Cu") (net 6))
 (segment (start 135.5 79.865) (end 133.635 78) (width 0.5) (layer "F.Cu") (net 6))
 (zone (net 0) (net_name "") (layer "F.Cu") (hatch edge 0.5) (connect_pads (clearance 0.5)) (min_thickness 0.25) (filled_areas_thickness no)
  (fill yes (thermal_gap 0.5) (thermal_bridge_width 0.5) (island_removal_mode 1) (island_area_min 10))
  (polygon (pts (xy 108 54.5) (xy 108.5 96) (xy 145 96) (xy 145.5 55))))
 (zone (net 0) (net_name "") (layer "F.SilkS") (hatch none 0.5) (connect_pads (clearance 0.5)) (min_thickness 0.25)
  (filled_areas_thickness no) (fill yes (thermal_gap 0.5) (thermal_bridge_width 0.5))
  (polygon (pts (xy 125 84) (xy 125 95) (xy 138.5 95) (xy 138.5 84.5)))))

